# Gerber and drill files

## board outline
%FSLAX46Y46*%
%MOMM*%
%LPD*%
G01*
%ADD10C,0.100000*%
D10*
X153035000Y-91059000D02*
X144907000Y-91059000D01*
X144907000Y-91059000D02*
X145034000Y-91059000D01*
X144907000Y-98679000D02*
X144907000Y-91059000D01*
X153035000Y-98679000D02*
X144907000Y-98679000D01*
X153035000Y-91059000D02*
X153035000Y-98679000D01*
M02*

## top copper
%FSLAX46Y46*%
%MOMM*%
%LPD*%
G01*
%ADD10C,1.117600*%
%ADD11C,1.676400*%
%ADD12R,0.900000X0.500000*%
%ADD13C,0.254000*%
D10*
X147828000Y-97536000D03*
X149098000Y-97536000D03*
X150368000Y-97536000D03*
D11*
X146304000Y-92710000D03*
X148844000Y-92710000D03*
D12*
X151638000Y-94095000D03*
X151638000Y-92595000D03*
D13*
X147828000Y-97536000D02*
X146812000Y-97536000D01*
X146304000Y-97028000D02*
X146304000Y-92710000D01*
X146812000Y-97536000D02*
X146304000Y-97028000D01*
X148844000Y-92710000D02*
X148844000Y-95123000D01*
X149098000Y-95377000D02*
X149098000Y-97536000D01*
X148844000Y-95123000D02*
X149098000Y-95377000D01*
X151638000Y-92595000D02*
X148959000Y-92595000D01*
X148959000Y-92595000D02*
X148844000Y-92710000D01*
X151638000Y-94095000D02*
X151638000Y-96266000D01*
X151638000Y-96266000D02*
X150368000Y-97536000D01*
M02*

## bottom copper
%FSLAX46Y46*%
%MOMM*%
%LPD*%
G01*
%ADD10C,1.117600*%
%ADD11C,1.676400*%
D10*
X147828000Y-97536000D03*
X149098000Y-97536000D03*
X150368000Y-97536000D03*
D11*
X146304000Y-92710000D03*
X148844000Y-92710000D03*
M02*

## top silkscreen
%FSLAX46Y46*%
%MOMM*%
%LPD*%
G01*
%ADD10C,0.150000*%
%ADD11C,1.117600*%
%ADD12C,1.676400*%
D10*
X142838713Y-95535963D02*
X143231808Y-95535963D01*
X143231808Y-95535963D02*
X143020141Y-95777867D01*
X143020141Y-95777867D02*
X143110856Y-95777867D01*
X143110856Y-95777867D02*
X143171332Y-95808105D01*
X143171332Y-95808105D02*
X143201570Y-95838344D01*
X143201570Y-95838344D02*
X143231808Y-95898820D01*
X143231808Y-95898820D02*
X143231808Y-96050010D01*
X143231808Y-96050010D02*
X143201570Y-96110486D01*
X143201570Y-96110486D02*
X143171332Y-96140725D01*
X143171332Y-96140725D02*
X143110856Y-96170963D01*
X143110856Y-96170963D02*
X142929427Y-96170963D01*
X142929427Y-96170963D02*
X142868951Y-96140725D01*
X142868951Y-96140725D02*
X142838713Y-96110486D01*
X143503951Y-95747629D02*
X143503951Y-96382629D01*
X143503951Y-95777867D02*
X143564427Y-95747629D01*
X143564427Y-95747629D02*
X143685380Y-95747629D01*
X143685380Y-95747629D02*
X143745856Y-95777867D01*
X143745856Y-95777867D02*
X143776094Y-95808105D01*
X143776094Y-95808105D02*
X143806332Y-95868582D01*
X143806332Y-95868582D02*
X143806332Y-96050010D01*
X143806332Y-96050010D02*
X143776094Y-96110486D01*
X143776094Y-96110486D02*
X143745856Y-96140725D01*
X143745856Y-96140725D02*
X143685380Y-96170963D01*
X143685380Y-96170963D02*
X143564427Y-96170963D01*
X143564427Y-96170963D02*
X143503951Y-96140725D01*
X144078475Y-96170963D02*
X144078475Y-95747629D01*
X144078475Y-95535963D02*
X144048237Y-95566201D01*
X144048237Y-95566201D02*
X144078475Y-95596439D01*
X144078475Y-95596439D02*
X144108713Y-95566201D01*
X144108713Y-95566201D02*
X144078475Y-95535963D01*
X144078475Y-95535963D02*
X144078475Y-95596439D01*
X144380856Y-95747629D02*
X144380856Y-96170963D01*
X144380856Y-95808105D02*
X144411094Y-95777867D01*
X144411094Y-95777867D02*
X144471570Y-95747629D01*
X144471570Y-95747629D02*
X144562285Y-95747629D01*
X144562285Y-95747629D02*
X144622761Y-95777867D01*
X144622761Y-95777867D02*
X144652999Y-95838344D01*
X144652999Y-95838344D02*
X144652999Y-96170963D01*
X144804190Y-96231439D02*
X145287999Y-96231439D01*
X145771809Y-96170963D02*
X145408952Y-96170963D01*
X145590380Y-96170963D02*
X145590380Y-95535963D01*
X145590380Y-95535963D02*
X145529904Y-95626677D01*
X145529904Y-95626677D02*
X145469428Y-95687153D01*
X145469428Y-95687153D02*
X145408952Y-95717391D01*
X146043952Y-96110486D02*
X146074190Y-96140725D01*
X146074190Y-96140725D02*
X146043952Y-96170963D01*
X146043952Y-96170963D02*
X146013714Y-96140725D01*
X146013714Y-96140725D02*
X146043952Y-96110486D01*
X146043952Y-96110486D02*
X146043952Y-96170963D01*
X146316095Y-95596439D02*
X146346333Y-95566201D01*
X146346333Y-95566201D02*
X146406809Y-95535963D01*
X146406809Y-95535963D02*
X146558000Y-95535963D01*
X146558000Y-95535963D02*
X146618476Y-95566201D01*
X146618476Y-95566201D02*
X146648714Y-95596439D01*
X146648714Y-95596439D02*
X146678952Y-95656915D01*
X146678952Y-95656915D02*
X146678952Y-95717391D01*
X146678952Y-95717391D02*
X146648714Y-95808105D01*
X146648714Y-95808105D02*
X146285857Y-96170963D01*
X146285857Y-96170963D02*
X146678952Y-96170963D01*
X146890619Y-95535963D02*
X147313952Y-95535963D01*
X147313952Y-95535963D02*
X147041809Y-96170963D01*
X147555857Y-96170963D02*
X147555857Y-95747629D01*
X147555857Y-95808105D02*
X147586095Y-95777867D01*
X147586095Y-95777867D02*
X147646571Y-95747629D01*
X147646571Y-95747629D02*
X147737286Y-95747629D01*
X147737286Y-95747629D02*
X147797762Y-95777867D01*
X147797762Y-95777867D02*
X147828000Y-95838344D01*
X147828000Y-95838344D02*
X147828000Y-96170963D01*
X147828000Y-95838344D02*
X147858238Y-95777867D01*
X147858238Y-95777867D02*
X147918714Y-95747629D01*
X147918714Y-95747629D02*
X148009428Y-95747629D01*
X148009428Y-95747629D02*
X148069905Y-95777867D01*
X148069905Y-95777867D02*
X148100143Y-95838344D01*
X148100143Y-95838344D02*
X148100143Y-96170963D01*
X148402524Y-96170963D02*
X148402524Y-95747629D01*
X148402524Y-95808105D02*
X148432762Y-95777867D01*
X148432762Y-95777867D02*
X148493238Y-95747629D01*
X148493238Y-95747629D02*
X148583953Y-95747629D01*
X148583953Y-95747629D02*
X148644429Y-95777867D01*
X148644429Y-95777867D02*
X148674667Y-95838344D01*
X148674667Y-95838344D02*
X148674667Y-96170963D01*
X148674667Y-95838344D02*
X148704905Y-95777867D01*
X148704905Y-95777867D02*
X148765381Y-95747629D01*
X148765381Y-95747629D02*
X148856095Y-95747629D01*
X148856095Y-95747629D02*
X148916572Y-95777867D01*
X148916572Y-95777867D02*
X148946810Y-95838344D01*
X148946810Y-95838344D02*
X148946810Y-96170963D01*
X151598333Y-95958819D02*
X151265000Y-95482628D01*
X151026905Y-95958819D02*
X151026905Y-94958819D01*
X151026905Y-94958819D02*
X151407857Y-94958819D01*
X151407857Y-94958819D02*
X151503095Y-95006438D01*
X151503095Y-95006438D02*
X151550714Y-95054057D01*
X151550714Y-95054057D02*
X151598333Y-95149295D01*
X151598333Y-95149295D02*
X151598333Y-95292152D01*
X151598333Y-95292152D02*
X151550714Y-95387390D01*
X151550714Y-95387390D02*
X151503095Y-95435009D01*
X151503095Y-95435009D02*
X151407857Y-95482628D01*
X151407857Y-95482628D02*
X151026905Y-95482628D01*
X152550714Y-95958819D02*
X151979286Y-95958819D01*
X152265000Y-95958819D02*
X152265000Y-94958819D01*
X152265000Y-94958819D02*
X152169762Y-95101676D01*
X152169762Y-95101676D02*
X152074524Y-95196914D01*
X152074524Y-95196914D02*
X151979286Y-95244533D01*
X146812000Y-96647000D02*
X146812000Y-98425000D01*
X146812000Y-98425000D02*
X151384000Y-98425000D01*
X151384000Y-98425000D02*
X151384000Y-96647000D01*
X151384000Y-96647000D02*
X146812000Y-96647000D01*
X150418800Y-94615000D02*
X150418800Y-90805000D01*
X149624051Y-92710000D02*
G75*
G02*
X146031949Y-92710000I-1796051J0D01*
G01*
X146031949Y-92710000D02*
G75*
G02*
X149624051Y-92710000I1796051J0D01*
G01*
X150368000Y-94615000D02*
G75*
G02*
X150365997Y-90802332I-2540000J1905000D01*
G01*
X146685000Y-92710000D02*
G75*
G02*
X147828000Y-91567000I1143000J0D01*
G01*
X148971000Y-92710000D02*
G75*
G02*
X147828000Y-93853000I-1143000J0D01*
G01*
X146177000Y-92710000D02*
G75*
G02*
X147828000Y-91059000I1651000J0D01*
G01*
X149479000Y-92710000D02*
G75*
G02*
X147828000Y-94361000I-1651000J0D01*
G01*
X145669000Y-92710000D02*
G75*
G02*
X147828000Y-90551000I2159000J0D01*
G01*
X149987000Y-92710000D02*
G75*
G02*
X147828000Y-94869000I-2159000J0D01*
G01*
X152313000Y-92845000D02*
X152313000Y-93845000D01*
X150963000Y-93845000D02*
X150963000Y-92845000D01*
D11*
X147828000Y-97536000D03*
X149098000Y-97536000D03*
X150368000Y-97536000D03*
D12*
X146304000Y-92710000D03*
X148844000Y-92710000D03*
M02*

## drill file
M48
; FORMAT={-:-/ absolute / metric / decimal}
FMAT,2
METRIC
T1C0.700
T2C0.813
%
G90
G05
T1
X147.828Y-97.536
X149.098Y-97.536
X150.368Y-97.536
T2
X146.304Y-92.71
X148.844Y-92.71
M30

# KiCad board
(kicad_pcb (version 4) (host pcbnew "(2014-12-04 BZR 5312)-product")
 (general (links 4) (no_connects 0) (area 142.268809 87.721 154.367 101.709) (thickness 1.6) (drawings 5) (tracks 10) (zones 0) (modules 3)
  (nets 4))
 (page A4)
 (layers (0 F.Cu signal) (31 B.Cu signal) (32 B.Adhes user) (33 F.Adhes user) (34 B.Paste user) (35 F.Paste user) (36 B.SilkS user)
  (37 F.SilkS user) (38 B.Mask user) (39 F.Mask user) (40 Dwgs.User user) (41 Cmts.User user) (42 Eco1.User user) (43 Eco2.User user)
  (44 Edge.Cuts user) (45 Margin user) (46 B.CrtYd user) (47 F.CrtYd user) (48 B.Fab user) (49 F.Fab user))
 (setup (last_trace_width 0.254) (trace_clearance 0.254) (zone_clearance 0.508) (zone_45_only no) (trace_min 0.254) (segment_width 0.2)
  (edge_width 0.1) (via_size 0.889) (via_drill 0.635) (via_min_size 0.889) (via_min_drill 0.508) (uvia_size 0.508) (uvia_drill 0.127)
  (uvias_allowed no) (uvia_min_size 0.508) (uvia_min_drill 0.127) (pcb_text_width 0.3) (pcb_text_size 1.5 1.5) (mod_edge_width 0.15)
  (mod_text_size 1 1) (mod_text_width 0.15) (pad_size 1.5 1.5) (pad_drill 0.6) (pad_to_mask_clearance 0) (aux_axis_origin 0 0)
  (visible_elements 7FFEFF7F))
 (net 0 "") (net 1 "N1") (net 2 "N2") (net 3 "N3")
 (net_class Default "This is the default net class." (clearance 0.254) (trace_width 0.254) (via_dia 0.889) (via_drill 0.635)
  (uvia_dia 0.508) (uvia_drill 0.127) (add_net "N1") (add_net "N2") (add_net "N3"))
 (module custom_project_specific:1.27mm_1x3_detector (layer F.Cu) (at 149.098 97.536)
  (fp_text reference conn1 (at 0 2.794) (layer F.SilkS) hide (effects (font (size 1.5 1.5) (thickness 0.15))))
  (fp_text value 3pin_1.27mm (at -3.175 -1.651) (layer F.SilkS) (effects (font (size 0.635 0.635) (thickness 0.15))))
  (fp_line (start -2.286 -0.889) (end -2.286 0.889) (layer F.SilkS) (width 0.15))
  (fp_line (start -2.286 0.889) (end 2.286 0.889) (layer F.SilkS) (width 0.15))
  (fp_line (start 2.286 0.889) (end 2.286 -0.889) (layer F.SilkS) (width 0.15))
  (fp_line (start 2.286 -0.889) (end -2.286 -0.889) (layer F.SilkS) (width 0.15))
  (pad 1 thru_hole circle (at -1.27 0) (size 1.1176 1.1176) (drill 0.7) (layers *.Cu *.Mask F.SilkS) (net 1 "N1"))
  (pad 2 thru_hole circle (at 0 0) (size 1.1176 1.1176) (drill 0.7) (layers *.Cu *.Mask F.SilkS) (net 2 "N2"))
  (pad 3 thru_hole circle (at 1.27 0) (size 1.1176 1.1176) (drill 0.7) (layers *.Cu *.Mask F.SilkS) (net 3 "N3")))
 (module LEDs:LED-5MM (layer F.Cu) (at 147.574 92.71)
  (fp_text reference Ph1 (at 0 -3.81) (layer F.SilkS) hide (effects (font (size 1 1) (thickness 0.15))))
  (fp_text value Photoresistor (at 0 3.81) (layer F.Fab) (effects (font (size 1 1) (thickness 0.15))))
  (fp_line (start 2.8448 1.905) (end 2.8448 -1.905) (layer F.SilkS) (width 0.15))
  (fp_circle (center 0.254 0) (end -1.016 1.27) (layer F.SilkS) (width 0.15))
  (fp_arc (start 0.254 0) (end 2.794 1.905) (angle 286.2) (layer F.SilkS) (width 0.15))
  (fp_arc (start 0.254 0) (end -0.889 0) (angle 90) (layer F.SilkS) (width 0.15))
  (fp_arc (start 0.254 0) (end 1.397 0) (angle 90) (layer F.SilkS) (width 0.15))
  (fp_arc (start 0.254 0) (end -1.397 0) (angle 90) (layer F.SilkS) (width 0.15))
  (fp_arc (start 0.254 0) (end 1.905 0) (angle 90) (layer F.SilkS) (width 0.15))
  (fp_arc (start 0.254 0) (end -1.905 0) (angle 90) (layer F.SilkS) (width 0.15))
  (fp_arc (start 0.254 0) (end 2.413 0) (angle 90) (layer F.SilkS) (width 0.15))
  (pad 1 thru_hole circle (at -1.27 0) (size 1.6764 1.6764) (drill 0.8128) (layers *.Cu *.Mask F.SilkS) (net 1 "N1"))
  (pad 2 thru_hole circle (at 1.27 0) (size 1.6764 1.6764) (drill 0.8128) (layers *.Cu *.Mask F.SilkS) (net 2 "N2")))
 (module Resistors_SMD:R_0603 (layer F.Cu) (at 151.638 93.345 90)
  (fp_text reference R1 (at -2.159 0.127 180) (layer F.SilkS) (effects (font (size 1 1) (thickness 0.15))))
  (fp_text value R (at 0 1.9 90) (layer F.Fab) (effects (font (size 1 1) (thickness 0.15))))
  (fp_line (start 0.5 0.675) (end -0.5 0.675) (layer F.SilkS) (width 0.15))
  (fp_line (start -0.5 -0.675) (end 0.5 -0.675) (layer F.SilkS) (width 0.15))
  (pad 1 smd rect (at -0.75 0 90) (size 0.5 0.9) (layers F.Cu F.Paste F.Mask) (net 3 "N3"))
  (pad 2 smd rect (at 0.75 0 90) (size 0.5 0.9) (layers F.Cu F.Paste F.Mask) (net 2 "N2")))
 (gr_line (start 153.035 91.059) (end 144.907 91.059) (angle 90) (layer Edge.Cuts) (width 0.1))
 (gr_line (start 144.907 91.059) (end 145.034 91.059) (angle 90) (layer Edge.Cuts) (width 0.1))
 (gr_line (start 144.907 98.679) (end 144.907 91.059) (angle 90) (layer Edge.Cuts) (width 0.1))
 (gr_line (start 153.035 98.679) (end 144.907 98.679) (angle 90) (layer Edge.Cuts) (width 0.1))
 (gr_line (start 153.035 91.059) (end 153.035 98.679) (angle 90) (layer Edge.Cuts) (width 0.1))
 (segment (start 147.828 97.536) (end 146.812 97.536) (width 0.254) (layer F.Cu) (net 1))
 (segment (start 146.304 97.028) (end 146.304 92.71) (width 0.254) (layer F.Cu) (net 1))
 (segment (start 146.812 97.536) (end 146.304 97.028) (width 0.254) (layer F.Cu) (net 1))
 (segment (start 148.844 92.71) (end 148.844 95.123) (width 0.254) (layer F.Cu) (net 2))
 (segment (start 149.098 95.377) (end 149.098 97.536) (width 0.254) (layer F.Cu) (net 2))
 (segment (start 148.844 95.123) (end 149.098 95.377) (width 0.254) (layer F.Cu) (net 2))
 (segment (start 151.638 92.595) (end 148.959 92.595) (width 0.254) (layer F.Cu) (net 2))
 (segment (start 148.959 92.595) (end 148.844 92.71) (width 0.254) (layer F.Cu) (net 2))
 (segment (start 151.638 94.095) (end 151.638 96.266) (width 0.254) (layer F.Cu) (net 3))
 (segment (start 151.638 96.266) (end 150.368 97.536) (width 0.254) (layer F.Cu) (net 3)))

